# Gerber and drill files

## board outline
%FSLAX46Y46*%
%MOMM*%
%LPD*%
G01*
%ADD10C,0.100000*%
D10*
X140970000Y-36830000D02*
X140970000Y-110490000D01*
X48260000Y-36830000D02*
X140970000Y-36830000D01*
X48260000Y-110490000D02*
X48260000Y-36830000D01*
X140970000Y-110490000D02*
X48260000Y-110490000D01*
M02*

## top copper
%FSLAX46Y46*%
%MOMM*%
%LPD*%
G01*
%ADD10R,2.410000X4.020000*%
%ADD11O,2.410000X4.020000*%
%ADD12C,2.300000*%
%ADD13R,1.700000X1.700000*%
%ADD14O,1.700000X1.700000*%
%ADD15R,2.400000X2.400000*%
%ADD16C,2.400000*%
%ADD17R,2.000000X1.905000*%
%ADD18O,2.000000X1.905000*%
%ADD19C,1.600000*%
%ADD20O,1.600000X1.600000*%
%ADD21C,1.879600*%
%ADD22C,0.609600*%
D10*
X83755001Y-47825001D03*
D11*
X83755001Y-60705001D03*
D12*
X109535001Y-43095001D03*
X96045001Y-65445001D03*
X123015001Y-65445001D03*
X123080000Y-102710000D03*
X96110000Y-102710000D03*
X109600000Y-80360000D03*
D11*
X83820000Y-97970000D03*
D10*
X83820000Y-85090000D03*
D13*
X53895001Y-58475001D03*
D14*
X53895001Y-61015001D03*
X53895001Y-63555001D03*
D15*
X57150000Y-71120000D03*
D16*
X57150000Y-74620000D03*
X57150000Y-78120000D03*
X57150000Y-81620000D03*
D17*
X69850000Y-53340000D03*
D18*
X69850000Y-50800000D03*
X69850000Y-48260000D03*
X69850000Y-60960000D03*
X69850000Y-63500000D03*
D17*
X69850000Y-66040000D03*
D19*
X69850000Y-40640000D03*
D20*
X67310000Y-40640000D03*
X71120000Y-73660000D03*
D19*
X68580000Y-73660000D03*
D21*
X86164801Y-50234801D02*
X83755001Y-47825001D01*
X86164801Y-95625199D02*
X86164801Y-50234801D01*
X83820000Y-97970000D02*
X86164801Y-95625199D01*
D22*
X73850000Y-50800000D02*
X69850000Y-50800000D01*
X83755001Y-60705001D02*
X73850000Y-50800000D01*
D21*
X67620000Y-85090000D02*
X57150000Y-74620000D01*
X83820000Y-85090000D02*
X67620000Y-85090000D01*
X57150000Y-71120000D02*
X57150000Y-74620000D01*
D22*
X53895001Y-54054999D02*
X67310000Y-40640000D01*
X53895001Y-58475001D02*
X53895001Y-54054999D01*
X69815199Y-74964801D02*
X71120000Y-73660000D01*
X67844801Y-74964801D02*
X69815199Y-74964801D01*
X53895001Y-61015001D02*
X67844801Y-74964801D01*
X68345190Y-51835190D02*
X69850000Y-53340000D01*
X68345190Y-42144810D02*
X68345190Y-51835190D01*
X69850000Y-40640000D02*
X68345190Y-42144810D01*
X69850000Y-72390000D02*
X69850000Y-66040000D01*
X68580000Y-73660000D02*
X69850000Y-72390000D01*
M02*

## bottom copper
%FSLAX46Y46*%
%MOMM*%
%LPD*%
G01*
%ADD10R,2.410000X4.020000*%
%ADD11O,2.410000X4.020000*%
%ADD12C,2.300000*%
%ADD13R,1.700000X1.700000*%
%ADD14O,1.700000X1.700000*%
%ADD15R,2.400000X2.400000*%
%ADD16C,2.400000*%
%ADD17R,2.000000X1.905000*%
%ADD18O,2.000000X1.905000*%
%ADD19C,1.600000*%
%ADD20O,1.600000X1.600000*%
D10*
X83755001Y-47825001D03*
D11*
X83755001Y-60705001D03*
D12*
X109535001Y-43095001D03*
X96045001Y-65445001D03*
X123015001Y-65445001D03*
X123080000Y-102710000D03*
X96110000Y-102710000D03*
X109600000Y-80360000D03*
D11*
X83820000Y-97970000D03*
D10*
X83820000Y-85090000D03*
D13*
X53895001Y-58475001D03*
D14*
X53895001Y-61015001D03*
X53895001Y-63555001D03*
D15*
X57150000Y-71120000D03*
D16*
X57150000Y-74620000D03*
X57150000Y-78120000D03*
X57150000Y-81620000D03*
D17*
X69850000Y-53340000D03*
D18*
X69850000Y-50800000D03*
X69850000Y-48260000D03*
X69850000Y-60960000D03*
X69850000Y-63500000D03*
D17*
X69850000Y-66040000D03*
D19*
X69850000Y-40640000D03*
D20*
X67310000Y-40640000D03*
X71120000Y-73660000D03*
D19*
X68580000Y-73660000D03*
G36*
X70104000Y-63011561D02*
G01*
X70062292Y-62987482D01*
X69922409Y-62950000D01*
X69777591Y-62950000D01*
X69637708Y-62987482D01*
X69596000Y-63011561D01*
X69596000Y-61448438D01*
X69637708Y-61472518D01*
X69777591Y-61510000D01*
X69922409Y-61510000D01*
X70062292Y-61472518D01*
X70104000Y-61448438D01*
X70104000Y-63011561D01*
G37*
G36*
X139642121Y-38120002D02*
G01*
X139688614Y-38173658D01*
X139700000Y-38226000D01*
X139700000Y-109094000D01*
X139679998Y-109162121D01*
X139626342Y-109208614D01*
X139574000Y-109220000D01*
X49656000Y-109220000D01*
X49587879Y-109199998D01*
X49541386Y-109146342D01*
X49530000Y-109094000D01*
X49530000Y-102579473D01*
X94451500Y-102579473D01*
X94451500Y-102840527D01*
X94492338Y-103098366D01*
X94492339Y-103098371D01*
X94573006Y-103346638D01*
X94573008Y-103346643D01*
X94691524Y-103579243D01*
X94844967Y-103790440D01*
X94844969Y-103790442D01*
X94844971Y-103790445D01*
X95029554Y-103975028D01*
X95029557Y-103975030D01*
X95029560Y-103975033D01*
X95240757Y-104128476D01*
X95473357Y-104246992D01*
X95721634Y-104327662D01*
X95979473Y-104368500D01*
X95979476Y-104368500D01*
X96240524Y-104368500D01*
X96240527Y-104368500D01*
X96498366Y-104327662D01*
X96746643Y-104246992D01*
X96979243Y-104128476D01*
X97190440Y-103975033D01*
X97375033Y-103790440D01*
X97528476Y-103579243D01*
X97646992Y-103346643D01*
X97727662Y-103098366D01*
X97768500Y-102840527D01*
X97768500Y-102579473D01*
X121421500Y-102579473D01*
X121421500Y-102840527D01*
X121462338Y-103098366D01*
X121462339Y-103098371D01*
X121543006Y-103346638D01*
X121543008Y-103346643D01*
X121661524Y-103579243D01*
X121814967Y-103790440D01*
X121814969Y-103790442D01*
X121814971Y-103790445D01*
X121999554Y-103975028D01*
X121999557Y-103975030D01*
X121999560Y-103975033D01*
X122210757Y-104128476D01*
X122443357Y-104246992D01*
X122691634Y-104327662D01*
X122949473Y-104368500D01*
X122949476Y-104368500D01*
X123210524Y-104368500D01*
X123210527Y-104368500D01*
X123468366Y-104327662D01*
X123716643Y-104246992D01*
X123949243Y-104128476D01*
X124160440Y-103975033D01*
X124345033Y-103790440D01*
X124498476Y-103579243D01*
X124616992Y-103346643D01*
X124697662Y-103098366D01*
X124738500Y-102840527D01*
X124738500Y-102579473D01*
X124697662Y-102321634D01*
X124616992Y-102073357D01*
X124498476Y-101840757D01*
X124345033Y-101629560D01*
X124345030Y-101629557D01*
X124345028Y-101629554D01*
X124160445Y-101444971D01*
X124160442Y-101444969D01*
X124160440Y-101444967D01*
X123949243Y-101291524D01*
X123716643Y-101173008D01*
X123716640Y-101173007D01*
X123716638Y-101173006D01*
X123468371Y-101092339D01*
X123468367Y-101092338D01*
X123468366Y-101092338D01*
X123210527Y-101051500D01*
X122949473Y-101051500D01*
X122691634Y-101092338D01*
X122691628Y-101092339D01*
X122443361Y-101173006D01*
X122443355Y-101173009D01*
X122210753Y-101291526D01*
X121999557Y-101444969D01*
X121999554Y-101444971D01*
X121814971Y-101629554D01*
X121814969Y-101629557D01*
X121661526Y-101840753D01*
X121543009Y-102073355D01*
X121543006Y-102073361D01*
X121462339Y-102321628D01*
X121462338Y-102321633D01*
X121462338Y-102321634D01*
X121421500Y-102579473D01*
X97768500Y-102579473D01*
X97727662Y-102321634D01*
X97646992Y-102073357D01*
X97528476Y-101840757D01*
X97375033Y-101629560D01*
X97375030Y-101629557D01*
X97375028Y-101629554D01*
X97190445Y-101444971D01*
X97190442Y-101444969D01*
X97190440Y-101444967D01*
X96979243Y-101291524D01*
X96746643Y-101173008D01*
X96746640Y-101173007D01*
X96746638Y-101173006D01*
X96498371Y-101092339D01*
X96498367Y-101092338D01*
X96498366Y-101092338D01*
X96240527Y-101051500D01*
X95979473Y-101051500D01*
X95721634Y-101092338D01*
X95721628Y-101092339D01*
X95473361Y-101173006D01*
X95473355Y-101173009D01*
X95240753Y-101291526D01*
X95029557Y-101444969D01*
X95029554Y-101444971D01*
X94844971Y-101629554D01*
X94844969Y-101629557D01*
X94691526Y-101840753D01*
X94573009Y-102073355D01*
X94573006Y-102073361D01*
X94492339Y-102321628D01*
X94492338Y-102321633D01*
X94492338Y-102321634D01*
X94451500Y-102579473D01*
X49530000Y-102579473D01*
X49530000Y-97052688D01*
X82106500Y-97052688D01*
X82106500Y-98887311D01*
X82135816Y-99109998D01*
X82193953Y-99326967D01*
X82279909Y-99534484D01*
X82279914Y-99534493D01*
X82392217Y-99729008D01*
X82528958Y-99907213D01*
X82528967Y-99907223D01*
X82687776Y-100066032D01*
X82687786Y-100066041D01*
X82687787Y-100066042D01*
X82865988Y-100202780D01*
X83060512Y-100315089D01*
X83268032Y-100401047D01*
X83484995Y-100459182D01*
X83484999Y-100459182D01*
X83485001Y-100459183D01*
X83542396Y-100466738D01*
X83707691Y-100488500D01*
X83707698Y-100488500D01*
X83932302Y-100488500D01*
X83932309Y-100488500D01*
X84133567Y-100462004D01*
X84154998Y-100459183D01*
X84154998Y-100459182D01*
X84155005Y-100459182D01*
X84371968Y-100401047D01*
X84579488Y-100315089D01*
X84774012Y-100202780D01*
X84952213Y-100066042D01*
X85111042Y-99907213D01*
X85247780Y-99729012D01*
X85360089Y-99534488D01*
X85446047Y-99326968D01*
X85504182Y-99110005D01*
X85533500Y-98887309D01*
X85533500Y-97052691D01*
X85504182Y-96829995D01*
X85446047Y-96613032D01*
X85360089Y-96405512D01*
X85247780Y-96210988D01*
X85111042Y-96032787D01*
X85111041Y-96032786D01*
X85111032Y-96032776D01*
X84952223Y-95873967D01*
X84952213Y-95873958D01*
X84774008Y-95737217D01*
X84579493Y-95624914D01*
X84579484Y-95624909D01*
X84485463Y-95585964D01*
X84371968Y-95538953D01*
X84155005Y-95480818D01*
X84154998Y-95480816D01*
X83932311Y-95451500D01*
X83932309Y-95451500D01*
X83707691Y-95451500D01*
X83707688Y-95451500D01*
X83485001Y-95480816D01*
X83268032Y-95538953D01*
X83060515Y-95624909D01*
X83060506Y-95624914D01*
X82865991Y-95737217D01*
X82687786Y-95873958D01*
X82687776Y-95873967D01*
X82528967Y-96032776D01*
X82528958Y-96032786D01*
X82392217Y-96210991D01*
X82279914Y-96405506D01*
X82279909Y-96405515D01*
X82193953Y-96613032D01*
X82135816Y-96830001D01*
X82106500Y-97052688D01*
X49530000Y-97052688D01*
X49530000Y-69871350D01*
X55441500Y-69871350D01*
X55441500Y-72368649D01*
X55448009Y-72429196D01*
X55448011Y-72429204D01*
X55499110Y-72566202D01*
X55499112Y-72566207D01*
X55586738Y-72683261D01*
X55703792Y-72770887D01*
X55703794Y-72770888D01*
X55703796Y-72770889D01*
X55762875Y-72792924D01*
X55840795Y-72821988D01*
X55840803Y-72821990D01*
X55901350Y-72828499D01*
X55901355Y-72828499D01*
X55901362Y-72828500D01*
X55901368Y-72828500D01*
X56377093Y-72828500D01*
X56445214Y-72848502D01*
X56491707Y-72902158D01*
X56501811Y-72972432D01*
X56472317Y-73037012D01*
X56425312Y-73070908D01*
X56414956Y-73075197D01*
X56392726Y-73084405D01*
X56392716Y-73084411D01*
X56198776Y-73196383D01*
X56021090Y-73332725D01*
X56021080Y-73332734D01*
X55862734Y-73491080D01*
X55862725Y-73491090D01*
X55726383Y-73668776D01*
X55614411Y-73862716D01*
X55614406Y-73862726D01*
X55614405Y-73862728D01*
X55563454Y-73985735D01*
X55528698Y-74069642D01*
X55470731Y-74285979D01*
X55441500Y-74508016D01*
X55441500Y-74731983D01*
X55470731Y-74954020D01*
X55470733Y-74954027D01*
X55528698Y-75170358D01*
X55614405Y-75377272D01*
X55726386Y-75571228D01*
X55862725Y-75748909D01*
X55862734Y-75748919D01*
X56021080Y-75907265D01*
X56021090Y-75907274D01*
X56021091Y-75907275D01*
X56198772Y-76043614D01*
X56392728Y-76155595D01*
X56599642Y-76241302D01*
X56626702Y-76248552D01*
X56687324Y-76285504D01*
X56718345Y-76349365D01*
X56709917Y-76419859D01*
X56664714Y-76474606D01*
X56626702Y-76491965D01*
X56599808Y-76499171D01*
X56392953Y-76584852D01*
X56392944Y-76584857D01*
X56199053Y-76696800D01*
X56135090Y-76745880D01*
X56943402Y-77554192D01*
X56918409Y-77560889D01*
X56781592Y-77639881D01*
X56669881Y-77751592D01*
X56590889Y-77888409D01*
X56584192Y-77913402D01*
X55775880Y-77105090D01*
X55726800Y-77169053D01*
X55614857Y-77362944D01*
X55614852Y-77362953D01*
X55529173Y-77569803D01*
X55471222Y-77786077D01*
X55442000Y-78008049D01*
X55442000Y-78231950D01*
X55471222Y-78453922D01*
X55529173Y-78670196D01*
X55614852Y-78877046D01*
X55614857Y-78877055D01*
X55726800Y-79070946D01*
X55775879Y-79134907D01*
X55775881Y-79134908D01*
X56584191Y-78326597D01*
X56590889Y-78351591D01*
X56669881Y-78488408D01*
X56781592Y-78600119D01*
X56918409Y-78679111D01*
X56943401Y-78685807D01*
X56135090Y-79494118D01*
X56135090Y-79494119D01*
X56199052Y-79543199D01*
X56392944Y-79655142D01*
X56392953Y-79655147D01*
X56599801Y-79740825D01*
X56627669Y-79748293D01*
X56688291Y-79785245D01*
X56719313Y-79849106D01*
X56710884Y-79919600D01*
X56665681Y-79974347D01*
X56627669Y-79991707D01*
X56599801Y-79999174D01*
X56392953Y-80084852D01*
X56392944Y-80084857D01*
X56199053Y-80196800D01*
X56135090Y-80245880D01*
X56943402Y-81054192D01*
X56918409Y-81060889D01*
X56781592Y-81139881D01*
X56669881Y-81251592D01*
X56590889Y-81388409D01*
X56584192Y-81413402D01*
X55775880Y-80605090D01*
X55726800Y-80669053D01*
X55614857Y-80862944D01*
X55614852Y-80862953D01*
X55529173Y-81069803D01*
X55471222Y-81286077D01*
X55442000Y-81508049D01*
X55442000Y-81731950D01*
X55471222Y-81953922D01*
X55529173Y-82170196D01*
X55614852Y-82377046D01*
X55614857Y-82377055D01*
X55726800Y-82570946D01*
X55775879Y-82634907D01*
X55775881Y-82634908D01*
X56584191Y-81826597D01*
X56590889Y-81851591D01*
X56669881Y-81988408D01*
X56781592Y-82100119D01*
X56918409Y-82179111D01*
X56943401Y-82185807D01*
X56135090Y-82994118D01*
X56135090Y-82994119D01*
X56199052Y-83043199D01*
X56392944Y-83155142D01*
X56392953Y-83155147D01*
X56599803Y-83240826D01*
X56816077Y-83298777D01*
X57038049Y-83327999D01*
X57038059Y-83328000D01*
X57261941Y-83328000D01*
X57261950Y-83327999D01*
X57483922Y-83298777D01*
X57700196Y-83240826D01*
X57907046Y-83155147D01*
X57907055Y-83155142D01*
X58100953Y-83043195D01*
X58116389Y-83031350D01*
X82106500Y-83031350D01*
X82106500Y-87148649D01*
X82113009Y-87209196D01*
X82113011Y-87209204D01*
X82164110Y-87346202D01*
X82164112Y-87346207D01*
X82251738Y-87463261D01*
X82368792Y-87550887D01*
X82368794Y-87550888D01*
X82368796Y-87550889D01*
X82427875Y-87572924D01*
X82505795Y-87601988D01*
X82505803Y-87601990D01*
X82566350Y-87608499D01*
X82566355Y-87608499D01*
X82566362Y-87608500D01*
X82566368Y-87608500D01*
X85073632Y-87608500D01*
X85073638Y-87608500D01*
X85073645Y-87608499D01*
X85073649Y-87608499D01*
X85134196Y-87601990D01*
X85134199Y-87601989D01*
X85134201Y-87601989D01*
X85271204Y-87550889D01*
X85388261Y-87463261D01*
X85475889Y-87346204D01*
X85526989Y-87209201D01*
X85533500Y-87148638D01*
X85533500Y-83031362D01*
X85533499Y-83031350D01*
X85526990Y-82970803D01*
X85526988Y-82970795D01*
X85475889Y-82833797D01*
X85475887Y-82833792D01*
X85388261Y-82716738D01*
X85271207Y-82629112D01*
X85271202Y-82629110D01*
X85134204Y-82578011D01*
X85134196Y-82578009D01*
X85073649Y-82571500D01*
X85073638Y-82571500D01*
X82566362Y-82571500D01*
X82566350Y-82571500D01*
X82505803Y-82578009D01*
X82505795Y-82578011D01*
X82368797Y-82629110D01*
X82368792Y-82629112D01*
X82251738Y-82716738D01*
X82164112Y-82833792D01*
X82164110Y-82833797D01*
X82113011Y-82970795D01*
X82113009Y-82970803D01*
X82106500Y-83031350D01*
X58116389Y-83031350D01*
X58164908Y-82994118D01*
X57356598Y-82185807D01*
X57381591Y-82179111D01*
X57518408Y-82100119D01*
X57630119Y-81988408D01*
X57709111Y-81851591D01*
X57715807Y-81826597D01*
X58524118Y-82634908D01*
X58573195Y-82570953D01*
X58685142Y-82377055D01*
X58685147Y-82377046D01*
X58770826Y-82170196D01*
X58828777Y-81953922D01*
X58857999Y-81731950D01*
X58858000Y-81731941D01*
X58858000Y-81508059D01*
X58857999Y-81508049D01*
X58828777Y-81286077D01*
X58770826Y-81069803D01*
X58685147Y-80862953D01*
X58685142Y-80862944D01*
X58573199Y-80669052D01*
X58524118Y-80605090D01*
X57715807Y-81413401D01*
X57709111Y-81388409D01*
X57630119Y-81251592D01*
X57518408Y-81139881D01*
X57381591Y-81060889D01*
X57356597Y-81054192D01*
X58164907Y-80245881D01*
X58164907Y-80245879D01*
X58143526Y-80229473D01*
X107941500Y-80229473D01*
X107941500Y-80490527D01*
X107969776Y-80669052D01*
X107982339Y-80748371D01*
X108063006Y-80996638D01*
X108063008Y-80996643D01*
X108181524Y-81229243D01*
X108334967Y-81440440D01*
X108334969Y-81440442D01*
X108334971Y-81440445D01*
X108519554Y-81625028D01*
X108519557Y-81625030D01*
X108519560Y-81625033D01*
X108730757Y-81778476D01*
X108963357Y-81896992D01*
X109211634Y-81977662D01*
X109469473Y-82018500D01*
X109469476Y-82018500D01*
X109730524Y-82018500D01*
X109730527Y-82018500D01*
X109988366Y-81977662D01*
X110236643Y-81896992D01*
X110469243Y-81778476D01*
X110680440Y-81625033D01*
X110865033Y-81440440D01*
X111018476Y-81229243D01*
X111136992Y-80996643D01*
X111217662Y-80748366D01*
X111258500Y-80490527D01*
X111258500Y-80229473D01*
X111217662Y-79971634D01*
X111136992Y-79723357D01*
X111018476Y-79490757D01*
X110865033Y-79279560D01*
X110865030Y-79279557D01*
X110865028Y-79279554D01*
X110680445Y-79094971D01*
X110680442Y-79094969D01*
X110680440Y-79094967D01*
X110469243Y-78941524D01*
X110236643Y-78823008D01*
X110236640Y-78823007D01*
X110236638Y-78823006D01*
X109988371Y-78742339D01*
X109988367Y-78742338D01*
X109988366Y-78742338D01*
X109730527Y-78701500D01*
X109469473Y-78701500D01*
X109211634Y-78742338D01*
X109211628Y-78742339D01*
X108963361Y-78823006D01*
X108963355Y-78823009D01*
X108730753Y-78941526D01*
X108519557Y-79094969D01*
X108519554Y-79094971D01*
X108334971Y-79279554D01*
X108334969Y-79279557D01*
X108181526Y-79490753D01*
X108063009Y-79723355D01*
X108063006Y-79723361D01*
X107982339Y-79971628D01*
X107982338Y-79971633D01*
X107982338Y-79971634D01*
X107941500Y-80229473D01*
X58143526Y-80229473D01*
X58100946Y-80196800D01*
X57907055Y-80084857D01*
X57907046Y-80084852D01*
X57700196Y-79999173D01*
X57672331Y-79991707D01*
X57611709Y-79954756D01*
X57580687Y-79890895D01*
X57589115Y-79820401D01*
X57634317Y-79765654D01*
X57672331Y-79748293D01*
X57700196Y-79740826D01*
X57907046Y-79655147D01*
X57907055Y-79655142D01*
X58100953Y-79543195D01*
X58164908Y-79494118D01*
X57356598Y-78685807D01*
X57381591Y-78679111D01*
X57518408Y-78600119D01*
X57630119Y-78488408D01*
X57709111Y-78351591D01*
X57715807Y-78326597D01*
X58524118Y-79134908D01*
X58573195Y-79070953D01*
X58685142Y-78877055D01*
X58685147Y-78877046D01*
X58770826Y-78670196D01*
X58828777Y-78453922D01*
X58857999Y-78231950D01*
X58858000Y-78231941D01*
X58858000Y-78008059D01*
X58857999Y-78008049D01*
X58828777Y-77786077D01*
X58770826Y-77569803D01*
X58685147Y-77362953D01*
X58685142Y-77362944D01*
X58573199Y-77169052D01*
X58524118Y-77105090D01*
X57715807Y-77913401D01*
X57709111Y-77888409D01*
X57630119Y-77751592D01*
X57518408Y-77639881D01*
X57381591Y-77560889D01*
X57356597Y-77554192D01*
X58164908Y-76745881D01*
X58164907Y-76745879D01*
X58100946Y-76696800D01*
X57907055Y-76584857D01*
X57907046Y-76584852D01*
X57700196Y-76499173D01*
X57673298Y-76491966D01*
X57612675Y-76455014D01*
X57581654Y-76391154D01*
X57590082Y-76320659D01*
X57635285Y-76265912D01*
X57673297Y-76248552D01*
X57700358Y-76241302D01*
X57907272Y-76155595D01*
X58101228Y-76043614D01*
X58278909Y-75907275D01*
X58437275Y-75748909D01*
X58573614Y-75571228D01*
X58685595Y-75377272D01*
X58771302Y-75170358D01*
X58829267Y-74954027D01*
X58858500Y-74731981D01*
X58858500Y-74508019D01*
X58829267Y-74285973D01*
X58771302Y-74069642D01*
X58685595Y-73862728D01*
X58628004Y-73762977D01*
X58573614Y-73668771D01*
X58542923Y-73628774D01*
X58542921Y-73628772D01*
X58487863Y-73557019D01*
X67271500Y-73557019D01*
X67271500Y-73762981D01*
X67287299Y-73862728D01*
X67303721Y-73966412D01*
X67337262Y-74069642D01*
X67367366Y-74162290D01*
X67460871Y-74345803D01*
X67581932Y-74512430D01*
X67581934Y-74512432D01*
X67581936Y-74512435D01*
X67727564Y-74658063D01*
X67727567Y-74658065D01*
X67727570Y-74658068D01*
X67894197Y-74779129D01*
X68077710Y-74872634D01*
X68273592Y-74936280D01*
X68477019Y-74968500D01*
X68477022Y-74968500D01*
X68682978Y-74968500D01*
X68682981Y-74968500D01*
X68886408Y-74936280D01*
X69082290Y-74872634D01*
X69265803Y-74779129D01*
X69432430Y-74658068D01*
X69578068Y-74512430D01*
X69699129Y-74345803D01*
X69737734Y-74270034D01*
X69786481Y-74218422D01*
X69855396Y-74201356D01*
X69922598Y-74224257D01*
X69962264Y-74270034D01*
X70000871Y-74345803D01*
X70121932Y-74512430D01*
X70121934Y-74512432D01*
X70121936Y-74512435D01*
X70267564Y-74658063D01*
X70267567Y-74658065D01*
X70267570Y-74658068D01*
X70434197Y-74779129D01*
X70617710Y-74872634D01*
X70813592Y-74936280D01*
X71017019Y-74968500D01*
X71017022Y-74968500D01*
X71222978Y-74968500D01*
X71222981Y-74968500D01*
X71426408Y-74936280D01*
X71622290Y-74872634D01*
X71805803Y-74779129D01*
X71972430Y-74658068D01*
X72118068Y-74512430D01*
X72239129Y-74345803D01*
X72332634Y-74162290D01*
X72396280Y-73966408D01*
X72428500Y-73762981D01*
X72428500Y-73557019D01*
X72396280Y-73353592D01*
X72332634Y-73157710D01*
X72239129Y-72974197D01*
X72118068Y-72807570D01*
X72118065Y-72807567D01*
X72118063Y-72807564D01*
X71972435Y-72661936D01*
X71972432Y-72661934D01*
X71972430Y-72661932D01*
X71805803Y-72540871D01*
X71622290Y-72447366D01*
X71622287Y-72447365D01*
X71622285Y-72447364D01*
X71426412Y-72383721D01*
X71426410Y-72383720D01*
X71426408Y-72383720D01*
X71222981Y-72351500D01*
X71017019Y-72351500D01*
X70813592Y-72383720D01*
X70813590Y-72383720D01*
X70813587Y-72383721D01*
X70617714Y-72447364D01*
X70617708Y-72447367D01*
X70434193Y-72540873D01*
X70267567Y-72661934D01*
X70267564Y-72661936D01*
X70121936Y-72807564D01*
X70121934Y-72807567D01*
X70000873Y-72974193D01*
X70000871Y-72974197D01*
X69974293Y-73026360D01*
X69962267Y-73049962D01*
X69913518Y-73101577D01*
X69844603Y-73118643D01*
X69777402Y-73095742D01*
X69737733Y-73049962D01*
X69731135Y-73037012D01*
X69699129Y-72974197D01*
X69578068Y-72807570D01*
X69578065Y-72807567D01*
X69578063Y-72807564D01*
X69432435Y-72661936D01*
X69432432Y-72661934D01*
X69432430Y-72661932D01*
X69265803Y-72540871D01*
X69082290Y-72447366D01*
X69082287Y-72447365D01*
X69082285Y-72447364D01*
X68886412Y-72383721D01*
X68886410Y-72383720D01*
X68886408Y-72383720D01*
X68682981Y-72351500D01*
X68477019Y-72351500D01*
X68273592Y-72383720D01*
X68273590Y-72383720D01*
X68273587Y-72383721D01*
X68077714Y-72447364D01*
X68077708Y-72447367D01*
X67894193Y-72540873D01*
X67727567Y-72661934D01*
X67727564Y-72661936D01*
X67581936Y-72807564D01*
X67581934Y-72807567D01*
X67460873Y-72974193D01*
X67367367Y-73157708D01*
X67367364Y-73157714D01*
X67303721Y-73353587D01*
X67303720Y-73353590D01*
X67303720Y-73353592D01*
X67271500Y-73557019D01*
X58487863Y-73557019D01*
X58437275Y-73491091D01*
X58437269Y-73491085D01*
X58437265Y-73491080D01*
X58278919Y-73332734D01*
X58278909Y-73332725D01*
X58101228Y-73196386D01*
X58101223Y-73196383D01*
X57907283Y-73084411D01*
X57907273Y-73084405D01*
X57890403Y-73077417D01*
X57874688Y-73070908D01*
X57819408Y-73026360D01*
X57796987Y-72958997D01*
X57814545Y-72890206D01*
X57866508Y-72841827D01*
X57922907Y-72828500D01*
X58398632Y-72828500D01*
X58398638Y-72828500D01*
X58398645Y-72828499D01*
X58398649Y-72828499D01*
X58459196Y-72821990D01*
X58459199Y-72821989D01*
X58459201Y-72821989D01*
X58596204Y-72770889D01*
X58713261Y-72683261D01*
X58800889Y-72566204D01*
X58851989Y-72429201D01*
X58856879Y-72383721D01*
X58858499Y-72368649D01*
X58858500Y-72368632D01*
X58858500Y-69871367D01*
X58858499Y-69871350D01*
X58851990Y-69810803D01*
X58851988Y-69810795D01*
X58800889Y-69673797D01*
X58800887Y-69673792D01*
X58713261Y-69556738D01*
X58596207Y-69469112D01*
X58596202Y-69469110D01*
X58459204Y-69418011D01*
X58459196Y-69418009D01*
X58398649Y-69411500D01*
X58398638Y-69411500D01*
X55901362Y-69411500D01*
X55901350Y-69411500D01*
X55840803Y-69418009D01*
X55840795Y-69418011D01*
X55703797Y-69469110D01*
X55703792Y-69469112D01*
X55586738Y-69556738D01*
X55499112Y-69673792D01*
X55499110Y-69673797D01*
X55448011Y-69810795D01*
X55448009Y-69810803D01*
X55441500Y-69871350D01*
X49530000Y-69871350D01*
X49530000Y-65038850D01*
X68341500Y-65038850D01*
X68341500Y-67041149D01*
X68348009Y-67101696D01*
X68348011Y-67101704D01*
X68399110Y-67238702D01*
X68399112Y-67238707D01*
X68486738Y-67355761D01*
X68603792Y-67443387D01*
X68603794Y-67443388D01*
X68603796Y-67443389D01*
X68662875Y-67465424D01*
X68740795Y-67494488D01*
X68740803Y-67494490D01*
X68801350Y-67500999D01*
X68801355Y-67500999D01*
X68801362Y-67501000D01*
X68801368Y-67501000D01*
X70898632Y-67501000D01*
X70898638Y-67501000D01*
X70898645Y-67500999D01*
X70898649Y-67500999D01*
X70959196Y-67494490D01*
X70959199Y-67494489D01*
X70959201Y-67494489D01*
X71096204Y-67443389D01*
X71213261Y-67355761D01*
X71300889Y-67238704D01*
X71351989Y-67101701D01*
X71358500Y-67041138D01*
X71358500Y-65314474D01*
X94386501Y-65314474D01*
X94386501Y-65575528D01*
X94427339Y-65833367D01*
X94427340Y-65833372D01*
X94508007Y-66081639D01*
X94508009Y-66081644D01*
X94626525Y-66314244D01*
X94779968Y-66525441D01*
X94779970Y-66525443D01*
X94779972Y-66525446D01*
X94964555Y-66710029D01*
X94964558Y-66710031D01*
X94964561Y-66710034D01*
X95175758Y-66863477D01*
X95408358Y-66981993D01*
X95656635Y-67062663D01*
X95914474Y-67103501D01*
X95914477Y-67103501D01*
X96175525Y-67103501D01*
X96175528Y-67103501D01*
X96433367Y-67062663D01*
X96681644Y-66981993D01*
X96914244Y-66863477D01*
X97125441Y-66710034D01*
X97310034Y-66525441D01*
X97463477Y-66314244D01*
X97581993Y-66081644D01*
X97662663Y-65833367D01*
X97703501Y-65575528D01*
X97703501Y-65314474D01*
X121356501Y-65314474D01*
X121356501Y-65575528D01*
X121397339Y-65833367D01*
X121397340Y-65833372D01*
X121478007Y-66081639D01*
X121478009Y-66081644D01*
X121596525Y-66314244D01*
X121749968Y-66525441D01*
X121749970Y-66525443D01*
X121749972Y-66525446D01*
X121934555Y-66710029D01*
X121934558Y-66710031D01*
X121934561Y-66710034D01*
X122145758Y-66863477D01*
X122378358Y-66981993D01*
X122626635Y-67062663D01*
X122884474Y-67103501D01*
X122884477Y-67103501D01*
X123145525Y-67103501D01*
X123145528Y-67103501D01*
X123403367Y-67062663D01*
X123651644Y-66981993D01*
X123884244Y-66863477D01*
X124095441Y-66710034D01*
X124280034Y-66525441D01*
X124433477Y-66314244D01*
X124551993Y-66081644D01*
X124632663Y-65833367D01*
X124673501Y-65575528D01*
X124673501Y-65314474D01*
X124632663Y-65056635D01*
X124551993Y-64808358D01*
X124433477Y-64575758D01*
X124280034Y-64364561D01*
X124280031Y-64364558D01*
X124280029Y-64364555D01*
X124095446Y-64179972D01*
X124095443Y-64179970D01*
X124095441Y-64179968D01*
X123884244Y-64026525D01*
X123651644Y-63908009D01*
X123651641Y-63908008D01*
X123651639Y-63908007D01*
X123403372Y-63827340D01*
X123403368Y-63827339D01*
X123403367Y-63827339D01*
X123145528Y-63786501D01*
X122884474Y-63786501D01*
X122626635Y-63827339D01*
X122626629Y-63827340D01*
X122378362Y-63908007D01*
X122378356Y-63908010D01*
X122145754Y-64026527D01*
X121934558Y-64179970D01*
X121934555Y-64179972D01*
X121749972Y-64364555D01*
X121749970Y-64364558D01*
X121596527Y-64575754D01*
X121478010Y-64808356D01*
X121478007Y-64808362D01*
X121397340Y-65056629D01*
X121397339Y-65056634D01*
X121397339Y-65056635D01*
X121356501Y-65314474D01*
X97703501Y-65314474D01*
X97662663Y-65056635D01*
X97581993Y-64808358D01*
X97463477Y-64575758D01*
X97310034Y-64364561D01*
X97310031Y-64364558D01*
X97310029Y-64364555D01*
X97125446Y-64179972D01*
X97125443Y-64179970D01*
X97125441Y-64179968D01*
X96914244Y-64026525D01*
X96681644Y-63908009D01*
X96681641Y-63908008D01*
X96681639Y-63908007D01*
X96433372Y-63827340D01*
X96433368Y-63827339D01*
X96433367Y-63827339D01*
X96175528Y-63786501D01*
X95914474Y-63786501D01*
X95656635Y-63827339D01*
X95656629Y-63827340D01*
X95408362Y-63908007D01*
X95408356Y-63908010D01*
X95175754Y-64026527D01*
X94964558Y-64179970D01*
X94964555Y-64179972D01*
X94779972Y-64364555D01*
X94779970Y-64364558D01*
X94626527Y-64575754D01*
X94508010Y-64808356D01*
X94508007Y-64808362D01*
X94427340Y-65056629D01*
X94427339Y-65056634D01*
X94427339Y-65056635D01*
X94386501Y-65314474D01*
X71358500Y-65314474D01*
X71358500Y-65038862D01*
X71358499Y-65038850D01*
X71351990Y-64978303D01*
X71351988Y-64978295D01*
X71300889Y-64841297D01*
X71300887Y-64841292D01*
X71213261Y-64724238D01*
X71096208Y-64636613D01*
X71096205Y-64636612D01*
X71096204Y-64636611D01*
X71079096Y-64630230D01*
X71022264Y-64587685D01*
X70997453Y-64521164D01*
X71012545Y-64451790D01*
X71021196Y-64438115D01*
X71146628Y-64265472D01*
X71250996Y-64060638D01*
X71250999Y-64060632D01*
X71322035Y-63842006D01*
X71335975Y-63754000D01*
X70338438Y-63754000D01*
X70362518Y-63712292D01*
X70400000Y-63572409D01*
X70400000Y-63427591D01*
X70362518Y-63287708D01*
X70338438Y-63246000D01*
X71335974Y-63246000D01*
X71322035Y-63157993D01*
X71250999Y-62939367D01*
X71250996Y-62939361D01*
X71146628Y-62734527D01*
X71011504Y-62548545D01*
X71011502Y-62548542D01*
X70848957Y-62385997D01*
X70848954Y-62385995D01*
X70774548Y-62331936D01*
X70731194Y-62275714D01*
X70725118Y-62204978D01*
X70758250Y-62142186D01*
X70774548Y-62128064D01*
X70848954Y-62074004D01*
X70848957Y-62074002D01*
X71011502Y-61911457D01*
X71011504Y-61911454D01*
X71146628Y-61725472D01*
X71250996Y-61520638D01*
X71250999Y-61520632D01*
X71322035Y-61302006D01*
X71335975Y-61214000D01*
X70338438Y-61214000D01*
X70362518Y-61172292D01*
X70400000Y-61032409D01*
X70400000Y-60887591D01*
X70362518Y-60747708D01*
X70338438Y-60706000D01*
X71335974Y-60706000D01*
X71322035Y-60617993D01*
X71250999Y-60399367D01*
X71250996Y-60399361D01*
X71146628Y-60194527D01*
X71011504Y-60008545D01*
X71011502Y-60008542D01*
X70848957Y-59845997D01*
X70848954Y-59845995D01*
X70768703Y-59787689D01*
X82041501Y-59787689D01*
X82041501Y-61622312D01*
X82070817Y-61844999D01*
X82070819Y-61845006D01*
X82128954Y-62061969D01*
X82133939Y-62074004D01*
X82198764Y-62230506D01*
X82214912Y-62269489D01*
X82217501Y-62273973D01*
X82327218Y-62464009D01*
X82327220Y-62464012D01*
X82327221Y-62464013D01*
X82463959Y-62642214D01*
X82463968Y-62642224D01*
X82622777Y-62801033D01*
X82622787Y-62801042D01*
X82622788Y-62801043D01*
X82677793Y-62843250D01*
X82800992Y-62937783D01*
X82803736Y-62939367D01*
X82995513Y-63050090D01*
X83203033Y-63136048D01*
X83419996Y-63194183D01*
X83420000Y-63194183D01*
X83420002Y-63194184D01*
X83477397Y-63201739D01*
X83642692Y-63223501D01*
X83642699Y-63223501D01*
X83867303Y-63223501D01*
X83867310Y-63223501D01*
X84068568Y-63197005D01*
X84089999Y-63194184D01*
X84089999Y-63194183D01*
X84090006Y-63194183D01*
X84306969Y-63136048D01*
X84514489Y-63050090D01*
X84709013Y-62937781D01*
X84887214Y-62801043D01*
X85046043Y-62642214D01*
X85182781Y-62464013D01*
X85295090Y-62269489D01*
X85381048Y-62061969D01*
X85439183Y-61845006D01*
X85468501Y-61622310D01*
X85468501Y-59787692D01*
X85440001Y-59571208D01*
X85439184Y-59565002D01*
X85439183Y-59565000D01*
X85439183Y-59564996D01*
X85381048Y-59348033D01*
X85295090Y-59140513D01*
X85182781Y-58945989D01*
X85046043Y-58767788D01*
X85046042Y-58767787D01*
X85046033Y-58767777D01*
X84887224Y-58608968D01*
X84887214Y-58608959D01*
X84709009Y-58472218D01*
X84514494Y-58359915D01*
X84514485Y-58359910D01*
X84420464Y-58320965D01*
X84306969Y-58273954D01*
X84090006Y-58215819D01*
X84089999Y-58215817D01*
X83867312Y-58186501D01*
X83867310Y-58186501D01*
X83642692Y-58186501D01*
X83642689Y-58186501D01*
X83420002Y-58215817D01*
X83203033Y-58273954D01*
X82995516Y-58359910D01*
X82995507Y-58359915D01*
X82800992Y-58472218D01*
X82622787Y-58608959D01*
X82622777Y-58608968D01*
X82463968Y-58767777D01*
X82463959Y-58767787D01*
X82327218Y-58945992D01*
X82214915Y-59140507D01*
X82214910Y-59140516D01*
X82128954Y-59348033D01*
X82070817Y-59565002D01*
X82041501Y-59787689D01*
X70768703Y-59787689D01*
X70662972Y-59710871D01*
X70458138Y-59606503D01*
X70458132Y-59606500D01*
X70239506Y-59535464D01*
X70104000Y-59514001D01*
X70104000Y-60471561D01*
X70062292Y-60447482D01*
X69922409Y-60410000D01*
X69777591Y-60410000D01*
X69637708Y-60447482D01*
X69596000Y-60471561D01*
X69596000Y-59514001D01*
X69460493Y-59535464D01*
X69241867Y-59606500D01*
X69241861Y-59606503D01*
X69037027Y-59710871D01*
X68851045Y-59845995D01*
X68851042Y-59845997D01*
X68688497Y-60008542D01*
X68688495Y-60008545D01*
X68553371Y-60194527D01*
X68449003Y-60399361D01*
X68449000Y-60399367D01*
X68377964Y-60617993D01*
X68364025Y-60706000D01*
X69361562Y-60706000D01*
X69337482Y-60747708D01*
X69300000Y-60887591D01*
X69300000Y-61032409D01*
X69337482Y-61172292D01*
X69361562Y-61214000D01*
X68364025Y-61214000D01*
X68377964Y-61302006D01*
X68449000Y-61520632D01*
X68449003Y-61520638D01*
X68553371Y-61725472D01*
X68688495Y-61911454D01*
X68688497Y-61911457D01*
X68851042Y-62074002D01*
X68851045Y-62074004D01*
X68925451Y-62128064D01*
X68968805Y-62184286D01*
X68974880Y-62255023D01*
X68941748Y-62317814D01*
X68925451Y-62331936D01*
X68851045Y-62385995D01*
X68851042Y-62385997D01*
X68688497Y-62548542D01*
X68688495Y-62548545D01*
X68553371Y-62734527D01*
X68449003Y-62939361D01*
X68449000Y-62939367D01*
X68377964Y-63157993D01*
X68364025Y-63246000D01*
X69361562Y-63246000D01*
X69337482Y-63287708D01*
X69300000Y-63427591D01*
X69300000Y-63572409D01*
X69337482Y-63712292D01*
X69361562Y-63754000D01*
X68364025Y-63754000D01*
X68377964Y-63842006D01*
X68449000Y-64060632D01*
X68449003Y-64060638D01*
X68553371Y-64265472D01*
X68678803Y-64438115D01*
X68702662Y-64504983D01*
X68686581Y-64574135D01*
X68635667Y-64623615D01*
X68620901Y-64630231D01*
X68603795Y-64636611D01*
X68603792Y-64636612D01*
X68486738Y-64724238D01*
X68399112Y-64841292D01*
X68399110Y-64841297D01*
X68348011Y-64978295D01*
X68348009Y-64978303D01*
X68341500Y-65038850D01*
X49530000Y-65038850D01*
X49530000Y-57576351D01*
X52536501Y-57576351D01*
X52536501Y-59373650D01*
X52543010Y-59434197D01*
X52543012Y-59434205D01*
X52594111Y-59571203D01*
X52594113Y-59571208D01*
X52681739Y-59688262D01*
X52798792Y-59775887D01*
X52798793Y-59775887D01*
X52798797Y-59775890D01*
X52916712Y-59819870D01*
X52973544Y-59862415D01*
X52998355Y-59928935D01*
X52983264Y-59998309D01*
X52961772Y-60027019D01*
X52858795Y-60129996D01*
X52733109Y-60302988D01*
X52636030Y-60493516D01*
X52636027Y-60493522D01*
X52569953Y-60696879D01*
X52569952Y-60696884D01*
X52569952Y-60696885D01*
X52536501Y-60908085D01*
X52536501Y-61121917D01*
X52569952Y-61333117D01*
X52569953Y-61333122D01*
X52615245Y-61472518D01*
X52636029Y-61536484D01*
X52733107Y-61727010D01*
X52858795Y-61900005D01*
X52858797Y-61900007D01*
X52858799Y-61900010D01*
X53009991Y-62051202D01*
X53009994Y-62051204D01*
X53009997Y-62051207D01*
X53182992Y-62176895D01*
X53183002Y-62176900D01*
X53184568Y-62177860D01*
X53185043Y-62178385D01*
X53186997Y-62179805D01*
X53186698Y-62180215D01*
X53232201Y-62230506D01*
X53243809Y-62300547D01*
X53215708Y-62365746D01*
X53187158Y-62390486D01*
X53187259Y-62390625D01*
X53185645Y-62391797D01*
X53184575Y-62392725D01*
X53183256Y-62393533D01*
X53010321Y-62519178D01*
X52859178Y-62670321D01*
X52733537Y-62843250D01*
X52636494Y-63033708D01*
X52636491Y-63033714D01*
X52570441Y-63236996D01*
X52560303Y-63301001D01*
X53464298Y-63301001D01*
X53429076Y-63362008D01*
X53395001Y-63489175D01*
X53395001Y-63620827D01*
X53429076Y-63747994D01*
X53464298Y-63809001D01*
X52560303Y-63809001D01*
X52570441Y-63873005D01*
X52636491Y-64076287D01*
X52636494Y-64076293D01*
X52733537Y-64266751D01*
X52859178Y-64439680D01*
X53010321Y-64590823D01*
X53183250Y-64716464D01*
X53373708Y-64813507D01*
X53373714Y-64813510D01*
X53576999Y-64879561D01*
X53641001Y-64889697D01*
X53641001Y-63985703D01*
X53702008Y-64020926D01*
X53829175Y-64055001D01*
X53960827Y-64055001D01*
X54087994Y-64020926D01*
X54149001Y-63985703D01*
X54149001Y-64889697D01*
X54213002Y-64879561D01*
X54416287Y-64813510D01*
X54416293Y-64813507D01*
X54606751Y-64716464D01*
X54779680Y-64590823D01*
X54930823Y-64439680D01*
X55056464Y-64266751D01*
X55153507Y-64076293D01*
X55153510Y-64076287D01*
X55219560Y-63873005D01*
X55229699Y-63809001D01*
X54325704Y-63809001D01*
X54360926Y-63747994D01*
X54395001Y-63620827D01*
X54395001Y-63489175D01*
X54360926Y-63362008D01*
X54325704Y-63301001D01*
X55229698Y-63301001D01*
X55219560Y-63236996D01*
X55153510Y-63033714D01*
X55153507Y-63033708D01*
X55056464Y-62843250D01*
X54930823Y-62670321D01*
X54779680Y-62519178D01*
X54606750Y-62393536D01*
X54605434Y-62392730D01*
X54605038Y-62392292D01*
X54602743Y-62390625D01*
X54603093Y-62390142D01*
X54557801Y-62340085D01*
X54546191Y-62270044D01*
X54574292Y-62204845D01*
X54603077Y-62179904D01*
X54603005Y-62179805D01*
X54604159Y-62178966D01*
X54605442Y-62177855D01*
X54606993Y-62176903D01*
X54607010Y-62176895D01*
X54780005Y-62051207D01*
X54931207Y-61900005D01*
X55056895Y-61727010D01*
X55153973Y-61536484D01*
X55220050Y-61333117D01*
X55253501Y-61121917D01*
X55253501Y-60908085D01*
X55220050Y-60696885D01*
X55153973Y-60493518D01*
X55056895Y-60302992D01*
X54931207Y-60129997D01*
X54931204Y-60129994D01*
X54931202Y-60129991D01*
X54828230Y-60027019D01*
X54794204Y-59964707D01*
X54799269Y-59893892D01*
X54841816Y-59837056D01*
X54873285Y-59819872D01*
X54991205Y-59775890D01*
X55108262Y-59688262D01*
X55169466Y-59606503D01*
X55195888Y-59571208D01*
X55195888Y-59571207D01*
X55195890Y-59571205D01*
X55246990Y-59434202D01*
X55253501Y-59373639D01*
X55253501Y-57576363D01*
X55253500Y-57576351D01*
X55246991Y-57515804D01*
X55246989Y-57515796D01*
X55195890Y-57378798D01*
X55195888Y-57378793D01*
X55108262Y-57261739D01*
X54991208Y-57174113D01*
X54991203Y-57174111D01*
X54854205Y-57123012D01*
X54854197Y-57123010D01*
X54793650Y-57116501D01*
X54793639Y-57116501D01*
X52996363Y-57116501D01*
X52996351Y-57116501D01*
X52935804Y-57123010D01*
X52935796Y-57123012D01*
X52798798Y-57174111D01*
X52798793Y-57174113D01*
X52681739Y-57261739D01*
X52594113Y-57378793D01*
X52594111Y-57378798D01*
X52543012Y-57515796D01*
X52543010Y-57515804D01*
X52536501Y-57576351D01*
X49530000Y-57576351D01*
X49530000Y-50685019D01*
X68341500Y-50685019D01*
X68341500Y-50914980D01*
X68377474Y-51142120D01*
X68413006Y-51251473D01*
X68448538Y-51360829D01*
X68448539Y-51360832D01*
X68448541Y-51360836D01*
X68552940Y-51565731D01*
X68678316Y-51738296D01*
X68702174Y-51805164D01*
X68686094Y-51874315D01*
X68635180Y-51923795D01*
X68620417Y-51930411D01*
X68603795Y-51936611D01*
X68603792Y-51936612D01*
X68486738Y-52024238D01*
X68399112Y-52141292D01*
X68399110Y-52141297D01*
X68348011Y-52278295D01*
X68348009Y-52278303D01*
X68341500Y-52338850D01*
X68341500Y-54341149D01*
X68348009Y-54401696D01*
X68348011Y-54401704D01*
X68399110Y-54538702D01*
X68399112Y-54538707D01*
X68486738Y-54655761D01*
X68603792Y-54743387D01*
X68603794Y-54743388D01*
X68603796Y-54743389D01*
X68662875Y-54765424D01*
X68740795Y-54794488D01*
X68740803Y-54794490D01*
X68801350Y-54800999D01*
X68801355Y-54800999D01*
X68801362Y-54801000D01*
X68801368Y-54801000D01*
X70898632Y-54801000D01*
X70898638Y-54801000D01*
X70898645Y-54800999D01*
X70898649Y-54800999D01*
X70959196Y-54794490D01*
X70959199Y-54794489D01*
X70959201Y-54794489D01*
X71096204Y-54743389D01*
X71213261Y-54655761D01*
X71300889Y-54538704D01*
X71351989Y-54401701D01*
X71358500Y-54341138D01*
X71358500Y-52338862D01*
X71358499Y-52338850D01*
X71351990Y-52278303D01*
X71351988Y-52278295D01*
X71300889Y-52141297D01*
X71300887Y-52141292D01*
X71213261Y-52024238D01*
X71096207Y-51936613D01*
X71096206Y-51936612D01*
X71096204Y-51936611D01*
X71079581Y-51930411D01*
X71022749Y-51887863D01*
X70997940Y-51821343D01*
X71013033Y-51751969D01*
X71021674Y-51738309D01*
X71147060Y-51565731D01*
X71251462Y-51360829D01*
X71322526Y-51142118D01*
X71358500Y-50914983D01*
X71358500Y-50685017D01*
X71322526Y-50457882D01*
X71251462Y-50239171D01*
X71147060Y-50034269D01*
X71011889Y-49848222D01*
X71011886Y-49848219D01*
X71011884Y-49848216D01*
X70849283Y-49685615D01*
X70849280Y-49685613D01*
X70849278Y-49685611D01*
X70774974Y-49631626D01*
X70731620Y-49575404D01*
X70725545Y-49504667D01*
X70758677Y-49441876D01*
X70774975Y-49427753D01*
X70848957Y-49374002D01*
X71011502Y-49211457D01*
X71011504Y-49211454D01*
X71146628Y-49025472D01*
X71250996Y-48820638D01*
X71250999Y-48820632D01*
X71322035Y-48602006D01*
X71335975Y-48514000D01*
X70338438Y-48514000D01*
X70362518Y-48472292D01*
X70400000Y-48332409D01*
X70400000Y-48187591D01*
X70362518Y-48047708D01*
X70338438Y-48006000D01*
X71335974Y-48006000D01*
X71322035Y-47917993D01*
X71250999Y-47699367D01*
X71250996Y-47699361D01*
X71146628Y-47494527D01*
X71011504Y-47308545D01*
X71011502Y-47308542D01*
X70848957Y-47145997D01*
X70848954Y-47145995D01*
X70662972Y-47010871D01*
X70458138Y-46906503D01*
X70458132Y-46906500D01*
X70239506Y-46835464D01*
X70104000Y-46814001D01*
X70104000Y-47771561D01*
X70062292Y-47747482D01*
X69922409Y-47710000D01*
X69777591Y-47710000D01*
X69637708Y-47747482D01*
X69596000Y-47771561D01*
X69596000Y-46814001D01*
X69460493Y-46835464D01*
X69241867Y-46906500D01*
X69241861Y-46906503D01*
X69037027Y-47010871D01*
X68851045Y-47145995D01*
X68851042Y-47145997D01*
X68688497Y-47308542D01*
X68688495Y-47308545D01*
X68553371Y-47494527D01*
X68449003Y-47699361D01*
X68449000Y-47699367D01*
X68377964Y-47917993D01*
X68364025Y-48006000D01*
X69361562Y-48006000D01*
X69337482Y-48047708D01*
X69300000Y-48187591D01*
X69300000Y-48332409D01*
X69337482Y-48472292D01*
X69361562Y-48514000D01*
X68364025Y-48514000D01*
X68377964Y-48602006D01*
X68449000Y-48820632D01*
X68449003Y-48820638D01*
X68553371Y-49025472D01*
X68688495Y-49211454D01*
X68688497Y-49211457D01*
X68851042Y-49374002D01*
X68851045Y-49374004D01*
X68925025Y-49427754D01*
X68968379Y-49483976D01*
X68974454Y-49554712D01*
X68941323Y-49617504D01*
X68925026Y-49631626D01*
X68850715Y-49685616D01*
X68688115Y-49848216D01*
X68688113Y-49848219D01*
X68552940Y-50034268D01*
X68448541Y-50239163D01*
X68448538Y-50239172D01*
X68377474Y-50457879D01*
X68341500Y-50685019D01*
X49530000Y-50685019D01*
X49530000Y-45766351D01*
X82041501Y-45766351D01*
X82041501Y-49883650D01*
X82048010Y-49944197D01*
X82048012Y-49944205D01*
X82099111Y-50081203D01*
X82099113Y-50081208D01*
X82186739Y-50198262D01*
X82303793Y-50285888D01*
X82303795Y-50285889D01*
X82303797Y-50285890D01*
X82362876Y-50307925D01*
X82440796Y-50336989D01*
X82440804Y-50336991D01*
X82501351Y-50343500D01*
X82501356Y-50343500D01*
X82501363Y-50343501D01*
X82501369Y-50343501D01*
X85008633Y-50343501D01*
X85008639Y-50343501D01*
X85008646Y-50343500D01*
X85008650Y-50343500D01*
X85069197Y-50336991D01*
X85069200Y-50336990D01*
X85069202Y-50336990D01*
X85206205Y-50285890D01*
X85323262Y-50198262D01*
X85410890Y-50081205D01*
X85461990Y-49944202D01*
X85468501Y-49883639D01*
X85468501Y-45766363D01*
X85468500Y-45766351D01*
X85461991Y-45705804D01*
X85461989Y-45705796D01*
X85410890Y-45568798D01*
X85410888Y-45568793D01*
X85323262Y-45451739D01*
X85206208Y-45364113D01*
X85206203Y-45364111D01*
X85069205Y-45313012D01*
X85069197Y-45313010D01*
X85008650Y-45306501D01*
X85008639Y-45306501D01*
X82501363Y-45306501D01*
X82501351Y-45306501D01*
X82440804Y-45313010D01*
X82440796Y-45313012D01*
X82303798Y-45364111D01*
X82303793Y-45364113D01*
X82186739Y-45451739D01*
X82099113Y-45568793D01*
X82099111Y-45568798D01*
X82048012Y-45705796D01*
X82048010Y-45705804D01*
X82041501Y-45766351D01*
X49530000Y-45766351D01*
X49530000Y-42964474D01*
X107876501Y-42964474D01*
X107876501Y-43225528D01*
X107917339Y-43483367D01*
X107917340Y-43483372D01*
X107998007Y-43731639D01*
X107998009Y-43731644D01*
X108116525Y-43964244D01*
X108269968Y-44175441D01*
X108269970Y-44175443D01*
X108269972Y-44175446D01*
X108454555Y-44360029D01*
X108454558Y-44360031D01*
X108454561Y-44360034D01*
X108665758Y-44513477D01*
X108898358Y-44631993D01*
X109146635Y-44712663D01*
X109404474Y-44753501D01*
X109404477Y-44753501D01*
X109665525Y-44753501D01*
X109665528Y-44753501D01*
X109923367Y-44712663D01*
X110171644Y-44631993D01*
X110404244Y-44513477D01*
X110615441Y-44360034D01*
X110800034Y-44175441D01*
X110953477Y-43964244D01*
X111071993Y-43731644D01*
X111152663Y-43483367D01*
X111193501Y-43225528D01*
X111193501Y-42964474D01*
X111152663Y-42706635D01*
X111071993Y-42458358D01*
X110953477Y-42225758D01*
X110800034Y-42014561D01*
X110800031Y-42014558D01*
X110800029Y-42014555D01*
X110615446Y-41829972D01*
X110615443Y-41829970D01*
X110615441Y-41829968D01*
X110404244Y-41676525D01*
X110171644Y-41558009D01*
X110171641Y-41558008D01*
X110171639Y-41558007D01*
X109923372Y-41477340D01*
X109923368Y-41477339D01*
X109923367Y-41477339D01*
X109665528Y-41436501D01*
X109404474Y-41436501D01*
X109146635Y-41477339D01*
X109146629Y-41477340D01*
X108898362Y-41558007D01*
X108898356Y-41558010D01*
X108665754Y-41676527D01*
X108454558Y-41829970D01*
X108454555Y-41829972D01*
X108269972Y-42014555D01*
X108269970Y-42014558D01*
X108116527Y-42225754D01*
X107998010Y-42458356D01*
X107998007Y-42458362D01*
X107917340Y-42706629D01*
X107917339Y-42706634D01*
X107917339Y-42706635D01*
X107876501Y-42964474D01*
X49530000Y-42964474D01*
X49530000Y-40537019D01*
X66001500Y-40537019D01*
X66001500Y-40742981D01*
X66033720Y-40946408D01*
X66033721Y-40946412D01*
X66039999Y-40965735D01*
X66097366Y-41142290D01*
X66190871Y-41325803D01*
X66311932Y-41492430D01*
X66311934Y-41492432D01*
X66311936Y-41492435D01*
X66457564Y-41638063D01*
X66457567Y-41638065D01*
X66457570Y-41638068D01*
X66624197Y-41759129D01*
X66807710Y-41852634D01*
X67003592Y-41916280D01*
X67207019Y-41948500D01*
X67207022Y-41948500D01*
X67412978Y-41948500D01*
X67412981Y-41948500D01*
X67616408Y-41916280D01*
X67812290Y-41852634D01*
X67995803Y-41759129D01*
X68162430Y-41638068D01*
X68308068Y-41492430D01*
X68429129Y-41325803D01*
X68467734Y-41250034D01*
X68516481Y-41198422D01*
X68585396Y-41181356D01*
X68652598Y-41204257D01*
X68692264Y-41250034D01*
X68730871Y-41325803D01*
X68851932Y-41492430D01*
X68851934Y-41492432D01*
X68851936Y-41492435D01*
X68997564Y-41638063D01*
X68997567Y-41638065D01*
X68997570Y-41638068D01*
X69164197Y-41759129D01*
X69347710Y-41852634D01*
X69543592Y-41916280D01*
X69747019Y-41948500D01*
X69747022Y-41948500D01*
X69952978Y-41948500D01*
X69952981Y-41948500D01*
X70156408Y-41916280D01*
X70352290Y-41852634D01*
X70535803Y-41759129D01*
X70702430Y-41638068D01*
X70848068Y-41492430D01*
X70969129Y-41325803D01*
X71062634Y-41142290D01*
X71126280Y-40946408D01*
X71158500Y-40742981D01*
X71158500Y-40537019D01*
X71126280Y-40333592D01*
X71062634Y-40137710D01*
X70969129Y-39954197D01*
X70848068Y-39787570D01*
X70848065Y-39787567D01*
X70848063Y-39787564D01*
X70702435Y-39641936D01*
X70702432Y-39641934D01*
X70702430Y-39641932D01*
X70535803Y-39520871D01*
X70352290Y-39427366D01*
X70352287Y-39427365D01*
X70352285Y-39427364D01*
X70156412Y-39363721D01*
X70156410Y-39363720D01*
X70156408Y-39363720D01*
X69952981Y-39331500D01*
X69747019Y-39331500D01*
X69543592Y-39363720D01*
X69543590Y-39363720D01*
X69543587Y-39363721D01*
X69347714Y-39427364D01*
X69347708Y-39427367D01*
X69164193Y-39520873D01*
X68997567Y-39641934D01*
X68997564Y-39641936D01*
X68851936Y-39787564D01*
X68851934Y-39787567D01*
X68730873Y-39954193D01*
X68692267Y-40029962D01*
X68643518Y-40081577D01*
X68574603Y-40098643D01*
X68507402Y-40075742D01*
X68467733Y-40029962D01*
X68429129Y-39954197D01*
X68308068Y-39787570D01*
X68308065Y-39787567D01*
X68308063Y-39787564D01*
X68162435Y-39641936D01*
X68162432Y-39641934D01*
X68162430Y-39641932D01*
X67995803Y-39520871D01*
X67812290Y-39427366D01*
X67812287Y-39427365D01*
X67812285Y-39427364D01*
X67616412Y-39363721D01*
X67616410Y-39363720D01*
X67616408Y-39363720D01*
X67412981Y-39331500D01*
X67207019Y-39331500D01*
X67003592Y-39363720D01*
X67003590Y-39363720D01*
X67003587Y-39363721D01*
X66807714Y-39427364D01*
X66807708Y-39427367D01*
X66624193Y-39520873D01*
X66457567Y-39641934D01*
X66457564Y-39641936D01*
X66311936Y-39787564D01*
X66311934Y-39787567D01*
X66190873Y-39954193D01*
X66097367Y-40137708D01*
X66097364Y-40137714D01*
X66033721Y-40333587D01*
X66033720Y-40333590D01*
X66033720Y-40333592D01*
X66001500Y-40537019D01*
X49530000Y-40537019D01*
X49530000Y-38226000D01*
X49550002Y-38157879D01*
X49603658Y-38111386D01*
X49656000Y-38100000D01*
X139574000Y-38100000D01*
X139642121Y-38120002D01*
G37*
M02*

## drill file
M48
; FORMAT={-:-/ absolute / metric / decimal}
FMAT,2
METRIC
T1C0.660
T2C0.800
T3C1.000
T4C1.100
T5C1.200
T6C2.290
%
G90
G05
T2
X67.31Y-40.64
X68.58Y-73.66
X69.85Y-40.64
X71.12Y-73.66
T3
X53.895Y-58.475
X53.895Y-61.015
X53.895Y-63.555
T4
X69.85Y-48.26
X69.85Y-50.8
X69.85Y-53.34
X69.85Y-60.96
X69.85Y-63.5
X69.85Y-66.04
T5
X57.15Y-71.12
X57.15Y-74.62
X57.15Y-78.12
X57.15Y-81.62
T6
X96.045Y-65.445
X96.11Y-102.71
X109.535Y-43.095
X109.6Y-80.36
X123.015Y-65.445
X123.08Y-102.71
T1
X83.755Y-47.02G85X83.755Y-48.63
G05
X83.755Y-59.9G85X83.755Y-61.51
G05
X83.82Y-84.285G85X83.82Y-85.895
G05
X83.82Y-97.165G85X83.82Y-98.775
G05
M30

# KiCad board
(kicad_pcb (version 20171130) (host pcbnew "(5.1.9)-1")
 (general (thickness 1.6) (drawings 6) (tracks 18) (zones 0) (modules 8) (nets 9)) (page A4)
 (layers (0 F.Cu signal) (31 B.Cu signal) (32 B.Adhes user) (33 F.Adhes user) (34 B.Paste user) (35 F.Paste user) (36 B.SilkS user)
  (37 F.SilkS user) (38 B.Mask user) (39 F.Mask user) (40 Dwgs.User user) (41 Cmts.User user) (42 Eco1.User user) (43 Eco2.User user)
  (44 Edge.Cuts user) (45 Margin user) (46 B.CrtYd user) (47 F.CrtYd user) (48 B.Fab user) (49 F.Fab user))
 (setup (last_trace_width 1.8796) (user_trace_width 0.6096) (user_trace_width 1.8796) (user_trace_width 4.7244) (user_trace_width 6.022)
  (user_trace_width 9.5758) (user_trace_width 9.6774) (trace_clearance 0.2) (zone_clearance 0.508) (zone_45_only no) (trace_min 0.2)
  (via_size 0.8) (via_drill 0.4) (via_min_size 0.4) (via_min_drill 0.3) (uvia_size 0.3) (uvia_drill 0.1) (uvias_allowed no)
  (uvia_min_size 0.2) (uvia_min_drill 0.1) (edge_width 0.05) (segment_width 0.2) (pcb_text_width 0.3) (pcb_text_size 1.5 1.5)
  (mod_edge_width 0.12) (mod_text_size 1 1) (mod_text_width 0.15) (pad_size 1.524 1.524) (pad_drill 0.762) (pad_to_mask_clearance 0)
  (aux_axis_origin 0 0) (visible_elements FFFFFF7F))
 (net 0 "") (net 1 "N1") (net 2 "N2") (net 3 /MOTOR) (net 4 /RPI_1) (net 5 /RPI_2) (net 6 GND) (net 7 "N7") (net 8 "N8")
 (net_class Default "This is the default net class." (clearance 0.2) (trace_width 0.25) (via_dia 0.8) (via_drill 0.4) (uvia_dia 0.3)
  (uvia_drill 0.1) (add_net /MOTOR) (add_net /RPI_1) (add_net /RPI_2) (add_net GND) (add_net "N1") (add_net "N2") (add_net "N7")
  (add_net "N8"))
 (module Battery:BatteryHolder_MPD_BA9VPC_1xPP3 (layer F.Cu) (at 83.755001 47.825001)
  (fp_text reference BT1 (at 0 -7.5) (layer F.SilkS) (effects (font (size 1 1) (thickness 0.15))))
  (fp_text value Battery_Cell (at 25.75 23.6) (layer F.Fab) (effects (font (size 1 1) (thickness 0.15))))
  (pad 1 thru_hole rect (at 0 0) (size 2.41 4.02) (drill oval 0.66 2.27) (layers *.Cu *.Mask) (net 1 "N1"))
  (pad 2 thru_hole oval (at 0 12.88) (size 2.41 4.02) (drill oval 0.66 2.27) (layers *.Cu *.Mask) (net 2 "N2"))
  (pad "" np_thru_hole circle (at 25.78 -4.73) (size 2.3 2.3) (drill 2.29) (layers *.Cu *.Mask))
  (pad "" np_thru_hole circle (at 12.29 17.62) (size 2.3 2.3) (drill 2.29) (layers *.Cu *.Mask))
  (pad "" np_thru_hole circle (at 39.26 17.62) (size 2.3 2.3) (drill 2.29) (layers *.Cu *.Mask)))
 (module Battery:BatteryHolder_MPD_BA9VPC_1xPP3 (layer F.Cu) (at 83.82 85.09)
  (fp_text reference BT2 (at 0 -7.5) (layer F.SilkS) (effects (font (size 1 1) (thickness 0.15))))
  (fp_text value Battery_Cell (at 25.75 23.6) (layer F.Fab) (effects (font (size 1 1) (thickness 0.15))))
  (pad "" np_thru_hole circle (at 39.26 17.62) (size 2.3 2.3) (drill 2.29) (layers *.Cu *.Mask))
  (pad "" np_thru_hole circle (at 12.29 17.62) (size 2.3 2.3) (drill 2.29) (layers *.Cu *.Mask))
  (pad "" np_thru_hole circle (at 25.78 -4.73) (size 2.3 2.3) (drill 2.29) (layers *.Cu *.Mask))
  (pad 2 thru_hole oval (at 0 12.88) (size 2.41 4.02) (drill oval 0.66 2.27) (layers *.Cu *.Mask) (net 1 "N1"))
  (pad 1 thru_hole rect (at 0 0) (size 2.41 4.02) (drill oval 0.66 2.27) (layers *.Cu *.Mask) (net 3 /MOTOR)))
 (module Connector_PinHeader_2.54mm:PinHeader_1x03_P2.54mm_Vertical (layer F.Cu) (at 53.895001 58.475001)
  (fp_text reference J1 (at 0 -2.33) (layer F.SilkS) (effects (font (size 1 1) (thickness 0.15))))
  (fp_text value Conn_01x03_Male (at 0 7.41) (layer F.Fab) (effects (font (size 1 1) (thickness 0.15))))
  (pad 1 thru_hole rect (at 0 0) (size 1.7 1.7) (drill 1) (layers *.Cu *.Mask) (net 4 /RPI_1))
  (pad 2 thru_hole oval (at 0 2.54) (size 1.7 1.7) (drill 1) (layers *.Cu *.Mask) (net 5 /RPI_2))
  (pad 3 thru_hole oval (at 0 5.08) (size 1.7 1.7) (drill 1) (layers *.Cu *.Mask) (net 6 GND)))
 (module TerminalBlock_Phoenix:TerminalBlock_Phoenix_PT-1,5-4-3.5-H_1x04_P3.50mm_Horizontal (layer F.Cu) (at 57.15 71.12 270)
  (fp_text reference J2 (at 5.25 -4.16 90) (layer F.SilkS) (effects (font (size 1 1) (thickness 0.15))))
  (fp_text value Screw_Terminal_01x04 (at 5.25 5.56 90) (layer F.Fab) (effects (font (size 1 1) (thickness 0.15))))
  (pad 1 thru_hole rect (at 0 0 270) (size 2.4 2.4) (drill 1.2) (layers *.Cu *.Mask) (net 3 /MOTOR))
  (pad 2 thru_hole circle (at 3.5 0 270) (size 2.4 2.4) (drill 1.2) (layers *.Cu *.Mask) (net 3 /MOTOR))
  (pad 3 thru_hole circle (at 7 0 270) (size 2.4 2.4) (drill 1.2) (layers *.Cu *.Mask) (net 6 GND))
  (pad 4 thru_hole circle (at 10.5 0 270) (size 2.4 2.4) (drill 1.2) (layers *.Cu *.Mask) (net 6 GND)))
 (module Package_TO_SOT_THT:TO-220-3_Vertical (layer F.Cu) (at 69.85 53.34 90)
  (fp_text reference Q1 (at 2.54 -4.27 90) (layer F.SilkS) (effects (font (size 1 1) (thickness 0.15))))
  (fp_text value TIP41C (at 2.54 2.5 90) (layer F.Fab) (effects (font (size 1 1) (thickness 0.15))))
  (pad 1 thru_hole rect (at 0 0 90) (size 1.905 2) (drill 1.1) (layers *.Cu *.Mask) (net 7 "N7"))
  (pad 2 thru_hole oval (at 2.54 0 90) (size 1.905 2) (drill 1.1) (layers *.Cu *.Mask) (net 2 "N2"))
  (pad 3 thru_hole oval (at 5.08 0 90) (size 1.905 2) (drill 1.1) (layers *.Cu *.Mask) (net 6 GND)))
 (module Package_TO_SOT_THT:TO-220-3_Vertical (layer F.Cu) (at 69.85 66.04 90)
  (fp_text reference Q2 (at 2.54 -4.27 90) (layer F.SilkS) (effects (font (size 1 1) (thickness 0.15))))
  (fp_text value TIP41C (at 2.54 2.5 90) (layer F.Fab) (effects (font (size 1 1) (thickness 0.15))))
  (pad 3 thru_hole oval (at 5.08 0 90) (size 1.905 2) (drill 1.1) (layers *.Cu *.Mask) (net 6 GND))
  (pad 2 thru_hole oval (at 2.54 0 90) (size 1.905 2) (drill 1.1) (layers *.Cu *.Mask) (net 6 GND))
  (pad 1 thru_hole rect (at 0 0 90) (size 1.905 2) (drill 1.1) (layers *.Cu *.Mask) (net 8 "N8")))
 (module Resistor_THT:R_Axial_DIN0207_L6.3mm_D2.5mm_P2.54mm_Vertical (layer F.Cu) (at 69.85 40.64 180)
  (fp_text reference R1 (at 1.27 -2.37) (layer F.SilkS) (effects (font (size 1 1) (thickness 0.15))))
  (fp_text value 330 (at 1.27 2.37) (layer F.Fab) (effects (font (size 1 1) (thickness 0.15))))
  (pad 1 thru_hole circle (at 0 0 180) (size 1.6 1.6) (drill 0.8) (layers *.Cu *.Mask) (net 7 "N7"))
  (pad 2 thru_hole oval (at 2.54 0 180) (size 1.6 1.6) (drill 0.8) (layers *.Cu *.Mask) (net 4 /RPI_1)))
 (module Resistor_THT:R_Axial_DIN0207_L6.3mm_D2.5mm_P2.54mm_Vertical (layer F.Cu) (at 68.58 73.66)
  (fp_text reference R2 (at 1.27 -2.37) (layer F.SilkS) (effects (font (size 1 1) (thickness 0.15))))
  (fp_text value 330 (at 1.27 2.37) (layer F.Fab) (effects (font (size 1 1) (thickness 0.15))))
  (pad 2 thru_hole oval (at 2.54 0) (size 1.6 1.6) (drill 0.8) (layers *.Cu *.Mask) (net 5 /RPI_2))
  (pad 1 thru_hole circle (at 0 0) (size 1.6 1.6) (drill 0.8) (layers *.Cu *.Mask) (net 8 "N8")))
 (gr_line (start 140.97 36.83) (end 140.97 110.49) (layer Edge.Cuts) (width 0.1))
 (gr_line (start 48.26 36.83) (end 140.97 36.83) (layer Edge.Cuts) (width 0.1))
 (gr_line (start 48.26 110.49) (end 48.26 36.83) (layer Edge.Cuts) (width 0.1))
 (gr_line (start 140.97 110.49) (end 48.26 110.49) (layer Edge.Cuts) (width 0.1))
 (segment (start 86.164801 50.234801) (end 83.755001 47.825001) (width 1.8796) (layer F.Cu) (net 1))
 (segment (start 86.164801 95.625199) (end 86.164801 50.234801) (width 1.8796) (layer F.Cu) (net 1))
 (segment (start 83.82 97.97) (end 86.164801 95.625199) (width 1.8796) (layer F.Cu) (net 1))
 (segment (start 73.85 50.8) (end 69.85 50.8) (width 0.6096) (layer F.Cu) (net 2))
 (segment (start 83.755001 60.705001) (end 73.85 50.8) (width 0.6096) (layer F.Cu) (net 2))
 (segment (start 67.62 85.09) (end 57.15 74.62) (width 1.8796) (layer F.Cu) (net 3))
 (segment (start 83.82 85.09) (end 67.62 85.09) (width 1.8796) (layer F.Cu) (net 3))
 (segment (start 57.15 71.12) (end 57.15 74.62) (width 1.8796) (layer F.Cu) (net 3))
 (segment (start 53.895001 54.054999) (end 67.31 40.64) (width 0.6096) (layer F.Cu) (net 4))
 (segment (start 53.895001 58.475001) (end 53.895001 54.054999) (width 0.6096) (layer F.Cu) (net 4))
 (segment (start 69.815199 74.964801) (end 71.12 73.66) (width 0.6096) (layer F.Cu) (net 5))
 (segment (start 67.844801 74.964801) (end 69.815199 74.964801) (width 0.6096) (layer F.Cu) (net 5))
 (segment (start 53.895001 61.015001) (end 67.844801 74.964801) (width 0.6096) (layer F.Cu) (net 5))
 (segment (start 68.34519 51.83519) (end 69.85 53.34) (width 0.6096) (layer F.Cu) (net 7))
 (segment (start 68.34519 42.14481) (end 68.34519 51.83519) (width 0.6096) (layer F.Cu) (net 7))
 (segment (start 69.85 40.64) (end 68.34519 42.14481) (width 0.6096) (layer F.Cu) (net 7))
 (segment (start 69.85 72.39) (end 69.85 66.04) (width 0.6096) (layer F.Cu) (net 8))
 (segment (start 68.58 73.66) (end 69.85 72.39) (width 0.6096) (layer F.Cu) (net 8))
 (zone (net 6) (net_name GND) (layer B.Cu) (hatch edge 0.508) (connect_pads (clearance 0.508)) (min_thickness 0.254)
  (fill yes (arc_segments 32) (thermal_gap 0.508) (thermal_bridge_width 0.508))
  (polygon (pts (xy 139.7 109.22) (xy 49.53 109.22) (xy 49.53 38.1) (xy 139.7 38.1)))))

